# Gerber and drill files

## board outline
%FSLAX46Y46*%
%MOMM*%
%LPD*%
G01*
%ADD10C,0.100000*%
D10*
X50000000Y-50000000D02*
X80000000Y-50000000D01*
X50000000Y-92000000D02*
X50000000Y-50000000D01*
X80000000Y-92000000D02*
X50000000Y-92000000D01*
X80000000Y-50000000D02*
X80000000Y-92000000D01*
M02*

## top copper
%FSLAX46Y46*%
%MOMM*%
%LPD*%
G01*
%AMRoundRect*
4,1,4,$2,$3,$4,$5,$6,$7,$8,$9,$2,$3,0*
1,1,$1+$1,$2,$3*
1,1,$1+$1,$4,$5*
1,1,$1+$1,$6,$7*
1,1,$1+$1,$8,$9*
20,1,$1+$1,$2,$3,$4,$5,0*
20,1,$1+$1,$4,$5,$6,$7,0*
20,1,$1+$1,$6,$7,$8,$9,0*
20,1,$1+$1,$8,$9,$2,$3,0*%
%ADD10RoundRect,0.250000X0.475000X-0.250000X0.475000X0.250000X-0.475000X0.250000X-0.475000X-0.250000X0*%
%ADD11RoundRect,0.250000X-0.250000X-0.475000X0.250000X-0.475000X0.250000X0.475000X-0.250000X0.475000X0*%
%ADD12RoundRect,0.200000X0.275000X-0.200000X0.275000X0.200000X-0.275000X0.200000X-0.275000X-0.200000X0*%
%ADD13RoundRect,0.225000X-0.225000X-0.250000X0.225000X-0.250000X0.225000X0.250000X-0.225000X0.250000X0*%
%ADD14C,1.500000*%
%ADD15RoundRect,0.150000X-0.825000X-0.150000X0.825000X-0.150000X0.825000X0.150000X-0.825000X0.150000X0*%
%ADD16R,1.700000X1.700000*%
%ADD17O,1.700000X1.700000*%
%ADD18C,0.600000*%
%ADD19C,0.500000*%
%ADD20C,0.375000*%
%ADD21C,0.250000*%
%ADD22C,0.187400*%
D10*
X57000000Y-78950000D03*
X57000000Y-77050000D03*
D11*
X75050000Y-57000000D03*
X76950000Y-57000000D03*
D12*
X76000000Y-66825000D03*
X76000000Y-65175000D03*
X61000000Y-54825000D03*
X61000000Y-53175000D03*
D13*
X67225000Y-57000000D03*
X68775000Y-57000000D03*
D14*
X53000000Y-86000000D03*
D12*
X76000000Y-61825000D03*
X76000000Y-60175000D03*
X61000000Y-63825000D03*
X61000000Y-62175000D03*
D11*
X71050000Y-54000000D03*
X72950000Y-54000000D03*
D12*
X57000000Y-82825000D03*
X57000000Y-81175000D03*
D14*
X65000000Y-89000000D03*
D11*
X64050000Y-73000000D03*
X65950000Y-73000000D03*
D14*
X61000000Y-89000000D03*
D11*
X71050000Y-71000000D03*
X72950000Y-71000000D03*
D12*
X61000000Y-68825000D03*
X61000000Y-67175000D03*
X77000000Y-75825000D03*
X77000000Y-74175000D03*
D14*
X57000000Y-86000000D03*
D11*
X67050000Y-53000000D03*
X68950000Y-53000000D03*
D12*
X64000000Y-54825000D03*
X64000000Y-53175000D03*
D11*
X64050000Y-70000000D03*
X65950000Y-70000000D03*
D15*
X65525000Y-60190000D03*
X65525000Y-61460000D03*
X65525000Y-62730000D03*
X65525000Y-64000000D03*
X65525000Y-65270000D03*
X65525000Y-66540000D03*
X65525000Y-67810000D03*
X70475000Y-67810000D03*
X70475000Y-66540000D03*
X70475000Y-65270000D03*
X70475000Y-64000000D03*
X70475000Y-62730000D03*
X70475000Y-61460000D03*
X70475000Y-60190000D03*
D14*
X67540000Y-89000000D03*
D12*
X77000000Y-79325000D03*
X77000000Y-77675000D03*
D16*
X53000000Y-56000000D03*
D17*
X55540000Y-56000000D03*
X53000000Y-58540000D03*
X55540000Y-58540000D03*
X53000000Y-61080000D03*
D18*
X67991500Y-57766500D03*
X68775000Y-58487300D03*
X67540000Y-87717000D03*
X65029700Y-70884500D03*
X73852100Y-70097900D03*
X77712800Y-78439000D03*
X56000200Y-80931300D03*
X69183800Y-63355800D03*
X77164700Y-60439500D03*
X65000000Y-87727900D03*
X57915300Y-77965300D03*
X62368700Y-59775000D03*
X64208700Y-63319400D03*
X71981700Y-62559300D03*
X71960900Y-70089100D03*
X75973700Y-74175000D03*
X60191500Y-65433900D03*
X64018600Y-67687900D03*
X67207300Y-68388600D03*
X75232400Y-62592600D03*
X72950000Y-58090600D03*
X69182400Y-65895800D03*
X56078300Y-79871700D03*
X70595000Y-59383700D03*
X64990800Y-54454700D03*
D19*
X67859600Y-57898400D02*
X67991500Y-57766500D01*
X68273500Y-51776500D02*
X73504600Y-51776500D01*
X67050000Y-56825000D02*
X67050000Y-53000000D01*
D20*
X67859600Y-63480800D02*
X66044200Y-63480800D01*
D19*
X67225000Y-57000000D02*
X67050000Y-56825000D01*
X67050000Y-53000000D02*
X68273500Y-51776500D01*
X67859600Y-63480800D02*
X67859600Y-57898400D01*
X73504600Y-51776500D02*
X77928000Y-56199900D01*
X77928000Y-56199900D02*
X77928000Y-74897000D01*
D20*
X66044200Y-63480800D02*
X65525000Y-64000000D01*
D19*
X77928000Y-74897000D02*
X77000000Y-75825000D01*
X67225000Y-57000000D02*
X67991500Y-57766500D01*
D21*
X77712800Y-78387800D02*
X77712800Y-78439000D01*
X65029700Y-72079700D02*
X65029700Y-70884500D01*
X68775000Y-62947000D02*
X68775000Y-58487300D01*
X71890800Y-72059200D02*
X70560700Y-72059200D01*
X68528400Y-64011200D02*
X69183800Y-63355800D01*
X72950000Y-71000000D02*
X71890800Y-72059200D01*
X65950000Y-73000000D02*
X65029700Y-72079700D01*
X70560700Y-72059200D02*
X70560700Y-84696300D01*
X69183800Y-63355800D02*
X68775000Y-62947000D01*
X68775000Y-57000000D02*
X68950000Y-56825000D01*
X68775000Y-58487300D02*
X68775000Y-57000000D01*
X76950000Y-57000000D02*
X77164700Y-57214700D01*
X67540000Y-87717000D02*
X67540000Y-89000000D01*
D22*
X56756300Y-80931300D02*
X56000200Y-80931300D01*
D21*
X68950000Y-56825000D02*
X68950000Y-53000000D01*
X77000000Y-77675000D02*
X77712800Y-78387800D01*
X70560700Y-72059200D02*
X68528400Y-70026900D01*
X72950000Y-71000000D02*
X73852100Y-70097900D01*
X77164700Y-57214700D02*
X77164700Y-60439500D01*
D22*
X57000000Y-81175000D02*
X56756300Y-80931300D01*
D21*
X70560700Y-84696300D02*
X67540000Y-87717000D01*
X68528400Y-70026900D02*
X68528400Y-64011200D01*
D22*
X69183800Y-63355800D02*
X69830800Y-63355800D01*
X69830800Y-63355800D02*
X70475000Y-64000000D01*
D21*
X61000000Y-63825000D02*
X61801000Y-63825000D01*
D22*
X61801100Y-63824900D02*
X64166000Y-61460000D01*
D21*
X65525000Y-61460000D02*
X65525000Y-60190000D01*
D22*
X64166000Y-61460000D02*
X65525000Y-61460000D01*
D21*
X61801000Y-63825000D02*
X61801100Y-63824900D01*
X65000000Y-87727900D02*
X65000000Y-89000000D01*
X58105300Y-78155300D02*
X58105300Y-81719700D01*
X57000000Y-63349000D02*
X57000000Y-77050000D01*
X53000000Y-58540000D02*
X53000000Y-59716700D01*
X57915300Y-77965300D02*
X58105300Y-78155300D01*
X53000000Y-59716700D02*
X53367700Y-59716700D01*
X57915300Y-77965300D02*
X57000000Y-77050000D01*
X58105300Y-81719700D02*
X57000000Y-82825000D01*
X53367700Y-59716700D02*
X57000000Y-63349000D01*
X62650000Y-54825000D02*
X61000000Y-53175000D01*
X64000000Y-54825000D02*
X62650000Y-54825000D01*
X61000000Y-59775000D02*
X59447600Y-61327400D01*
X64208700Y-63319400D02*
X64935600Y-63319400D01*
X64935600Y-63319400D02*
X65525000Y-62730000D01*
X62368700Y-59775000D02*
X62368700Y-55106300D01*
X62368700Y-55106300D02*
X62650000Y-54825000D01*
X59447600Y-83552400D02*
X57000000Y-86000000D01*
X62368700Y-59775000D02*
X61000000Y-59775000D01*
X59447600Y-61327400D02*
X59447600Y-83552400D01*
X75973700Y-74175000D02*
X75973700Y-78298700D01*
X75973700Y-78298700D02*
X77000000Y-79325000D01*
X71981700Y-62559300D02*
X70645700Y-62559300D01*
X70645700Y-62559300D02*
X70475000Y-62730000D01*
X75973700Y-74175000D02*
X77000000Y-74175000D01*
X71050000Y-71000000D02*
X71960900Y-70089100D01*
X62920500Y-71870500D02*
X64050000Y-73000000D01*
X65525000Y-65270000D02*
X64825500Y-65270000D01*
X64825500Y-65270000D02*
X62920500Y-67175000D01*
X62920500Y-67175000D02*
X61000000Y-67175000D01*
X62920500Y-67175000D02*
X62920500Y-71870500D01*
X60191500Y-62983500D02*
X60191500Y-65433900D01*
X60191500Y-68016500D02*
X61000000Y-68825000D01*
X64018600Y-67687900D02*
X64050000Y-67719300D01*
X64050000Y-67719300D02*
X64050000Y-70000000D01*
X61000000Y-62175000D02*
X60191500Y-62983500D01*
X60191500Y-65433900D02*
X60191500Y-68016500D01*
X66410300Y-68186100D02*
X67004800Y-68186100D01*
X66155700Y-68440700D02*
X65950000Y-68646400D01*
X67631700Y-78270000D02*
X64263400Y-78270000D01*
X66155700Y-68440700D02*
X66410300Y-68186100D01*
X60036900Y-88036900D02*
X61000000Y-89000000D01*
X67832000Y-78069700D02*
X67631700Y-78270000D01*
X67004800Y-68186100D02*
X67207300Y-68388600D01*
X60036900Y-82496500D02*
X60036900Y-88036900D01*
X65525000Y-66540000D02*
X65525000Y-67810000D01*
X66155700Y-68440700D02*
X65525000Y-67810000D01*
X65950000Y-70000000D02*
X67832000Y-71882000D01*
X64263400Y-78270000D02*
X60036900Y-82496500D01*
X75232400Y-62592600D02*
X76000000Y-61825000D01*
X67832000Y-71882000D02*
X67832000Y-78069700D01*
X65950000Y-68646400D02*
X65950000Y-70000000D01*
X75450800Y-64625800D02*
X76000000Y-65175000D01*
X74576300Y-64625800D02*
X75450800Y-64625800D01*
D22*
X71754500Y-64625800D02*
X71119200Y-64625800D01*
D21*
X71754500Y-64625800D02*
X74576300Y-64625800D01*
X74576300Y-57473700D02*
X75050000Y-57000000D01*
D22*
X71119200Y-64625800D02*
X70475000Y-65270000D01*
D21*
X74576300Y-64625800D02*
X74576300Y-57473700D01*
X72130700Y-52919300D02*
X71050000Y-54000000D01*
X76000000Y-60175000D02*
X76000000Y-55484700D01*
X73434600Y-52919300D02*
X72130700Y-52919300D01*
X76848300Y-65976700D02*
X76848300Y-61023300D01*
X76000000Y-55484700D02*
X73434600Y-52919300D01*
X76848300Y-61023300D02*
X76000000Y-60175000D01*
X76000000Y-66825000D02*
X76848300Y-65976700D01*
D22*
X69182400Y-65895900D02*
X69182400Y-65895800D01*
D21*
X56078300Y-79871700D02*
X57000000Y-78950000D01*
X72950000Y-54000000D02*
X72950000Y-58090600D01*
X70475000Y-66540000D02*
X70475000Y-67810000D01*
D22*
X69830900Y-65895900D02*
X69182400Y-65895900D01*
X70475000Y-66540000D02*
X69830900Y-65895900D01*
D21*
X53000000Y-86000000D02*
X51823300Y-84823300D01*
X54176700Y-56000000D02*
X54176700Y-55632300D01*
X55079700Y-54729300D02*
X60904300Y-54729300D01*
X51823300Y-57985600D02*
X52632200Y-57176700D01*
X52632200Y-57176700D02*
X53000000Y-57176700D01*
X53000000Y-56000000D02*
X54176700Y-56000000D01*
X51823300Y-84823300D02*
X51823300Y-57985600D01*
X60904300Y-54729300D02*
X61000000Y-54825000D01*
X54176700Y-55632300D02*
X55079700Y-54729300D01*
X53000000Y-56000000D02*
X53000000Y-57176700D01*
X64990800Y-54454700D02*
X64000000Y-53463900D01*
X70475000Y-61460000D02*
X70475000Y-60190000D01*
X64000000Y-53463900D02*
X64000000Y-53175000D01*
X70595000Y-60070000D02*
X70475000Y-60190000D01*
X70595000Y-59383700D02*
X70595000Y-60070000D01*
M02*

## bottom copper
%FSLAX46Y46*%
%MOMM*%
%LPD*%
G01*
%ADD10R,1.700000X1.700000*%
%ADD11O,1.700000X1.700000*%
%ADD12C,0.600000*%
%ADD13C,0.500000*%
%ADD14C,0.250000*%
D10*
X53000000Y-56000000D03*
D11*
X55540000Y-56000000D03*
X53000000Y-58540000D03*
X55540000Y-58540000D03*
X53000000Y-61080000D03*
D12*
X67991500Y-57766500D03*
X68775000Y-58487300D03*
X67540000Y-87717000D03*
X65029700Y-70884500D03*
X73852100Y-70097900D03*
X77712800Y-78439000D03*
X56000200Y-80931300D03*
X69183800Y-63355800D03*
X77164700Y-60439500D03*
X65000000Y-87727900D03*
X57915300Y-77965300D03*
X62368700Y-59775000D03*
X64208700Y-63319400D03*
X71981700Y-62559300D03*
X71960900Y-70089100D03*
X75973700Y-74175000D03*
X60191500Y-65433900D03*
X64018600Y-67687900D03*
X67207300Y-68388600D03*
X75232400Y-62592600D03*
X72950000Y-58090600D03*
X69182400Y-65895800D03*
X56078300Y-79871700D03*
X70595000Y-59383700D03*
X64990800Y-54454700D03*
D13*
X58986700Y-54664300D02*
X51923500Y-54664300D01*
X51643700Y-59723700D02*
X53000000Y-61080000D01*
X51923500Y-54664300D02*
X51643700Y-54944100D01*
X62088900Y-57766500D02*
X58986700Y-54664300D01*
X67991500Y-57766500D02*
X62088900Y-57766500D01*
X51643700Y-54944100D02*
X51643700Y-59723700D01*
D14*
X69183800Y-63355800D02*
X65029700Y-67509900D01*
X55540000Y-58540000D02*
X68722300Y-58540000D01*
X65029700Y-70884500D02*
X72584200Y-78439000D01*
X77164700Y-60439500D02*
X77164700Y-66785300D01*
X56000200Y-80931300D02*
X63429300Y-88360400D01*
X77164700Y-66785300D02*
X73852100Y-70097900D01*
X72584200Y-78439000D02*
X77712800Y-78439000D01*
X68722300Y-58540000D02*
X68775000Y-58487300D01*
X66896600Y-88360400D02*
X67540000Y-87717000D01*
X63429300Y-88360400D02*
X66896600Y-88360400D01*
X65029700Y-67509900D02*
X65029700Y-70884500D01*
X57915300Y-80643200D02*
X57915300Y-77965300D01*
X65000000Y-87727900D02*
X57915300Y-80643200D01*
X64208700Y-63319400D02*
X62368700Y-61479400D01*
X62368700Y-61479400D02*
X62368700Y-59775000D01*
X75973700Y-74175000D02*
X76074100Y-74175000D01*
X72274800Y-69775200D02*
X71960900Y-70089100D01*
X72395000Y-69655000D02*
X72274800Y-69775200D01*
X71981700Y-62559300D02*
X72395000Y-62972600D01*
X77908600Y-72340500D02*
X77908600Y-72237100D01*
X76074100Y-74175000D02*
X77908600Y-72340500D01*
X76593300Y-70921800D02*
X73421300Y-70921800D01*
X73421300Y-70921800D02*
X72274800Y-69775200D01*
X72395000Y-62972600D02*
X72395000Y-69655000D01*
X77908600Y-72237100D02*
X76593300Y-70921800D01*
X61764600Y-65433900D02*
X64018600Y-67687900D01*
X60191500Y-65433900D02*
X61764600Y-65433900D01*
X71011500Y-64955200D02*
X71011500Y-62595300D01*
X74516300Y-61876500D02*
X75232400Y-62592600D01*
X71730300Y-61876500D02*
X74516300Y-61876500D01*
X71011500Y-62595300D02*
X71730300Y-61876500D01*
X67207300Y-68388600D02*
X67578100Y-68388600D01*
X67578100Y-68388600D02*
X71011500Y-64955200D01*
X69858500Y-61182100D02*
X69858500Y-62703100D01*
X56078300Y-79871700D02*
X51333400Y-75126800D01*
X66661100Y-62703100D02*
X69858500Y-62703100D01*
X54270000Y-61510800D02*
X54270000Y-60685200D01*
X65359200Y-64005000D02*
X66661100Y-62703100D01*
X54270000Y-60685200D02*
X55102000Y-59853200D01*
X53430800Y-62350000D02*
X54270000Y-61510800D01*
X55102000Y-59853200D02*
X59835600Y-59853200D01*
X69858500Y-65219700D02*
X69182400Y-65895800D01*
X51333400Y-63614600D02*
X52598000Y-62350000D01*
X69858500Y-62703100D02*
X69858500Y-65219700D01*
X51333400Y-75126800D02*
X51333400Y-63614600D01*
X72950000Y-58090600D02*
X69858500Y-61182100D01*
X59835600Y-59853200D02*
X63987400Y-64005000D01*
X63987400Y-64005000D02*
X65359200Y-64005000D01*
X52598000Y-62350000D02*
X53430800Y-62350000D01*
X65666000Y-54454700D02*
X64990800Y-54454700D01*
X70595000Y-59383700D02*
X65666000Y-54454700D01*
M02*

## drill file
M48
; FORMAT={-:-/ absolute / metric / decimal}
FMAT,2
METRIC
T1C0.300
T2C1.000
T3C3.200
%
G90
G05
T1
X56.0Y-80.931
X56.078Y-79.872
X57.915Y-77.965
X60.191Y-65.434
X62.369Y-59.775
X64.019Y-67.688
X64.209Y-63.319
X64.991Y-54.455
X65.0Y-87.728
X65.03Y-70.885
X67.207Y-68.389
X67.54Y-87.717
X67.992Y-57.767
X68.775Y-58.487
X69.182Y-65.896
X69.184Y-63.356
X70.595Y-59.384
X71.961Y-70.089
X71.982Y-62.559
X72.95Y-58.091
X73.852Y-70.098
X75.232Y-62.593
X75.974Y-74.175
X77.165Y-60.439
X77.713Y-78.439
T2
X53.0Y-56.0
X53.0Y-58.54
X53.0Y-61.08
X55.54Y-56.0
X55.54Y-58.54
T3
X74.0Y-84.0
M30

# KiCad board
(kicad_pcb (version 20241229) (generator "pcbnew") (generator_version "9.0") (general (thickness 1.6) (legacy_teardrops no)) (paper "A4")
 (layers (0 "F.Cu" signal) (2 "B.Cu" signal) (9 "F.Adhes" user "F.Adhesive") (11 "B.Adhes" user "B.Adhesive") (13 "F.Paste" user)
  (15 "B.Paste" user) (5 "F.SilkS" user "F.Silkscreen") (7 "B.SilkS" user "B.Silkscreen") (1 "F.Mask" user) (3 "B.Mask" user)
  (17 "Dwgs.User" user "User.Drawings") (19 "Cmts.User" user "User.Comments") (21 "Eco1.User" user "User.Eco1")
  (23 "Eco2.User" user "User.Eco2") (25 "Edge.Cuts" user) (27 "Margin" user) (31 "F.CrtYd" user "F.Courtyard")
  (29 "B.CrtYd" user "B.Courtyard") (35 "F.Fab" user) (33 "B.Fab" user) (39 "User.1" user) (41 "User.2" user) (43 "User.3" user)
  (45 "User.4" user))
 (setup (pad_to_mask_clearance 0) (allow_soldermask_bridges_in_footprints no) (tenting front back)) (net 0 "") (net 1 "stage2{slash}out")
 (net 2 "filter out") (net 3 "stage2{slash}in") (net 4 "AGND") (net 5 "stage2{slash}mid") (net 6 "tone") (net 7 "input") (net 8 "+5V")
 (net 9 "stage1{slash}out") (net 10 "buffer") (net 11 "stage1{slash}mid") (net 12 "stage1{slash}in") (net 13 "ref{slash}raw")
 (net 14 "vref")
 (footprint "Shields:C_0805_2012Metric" (layer "F.Cu") (at 57 78 90)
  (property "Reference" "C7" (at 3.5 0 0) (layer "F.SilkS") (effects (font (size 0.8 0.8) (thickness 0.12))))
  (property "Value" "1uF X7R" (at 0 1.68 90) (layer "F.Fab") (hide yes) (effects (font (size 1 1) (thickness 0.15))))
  (pad "1" smd roundrect (at -0.95 0 90) (size 1 1.45) (layers "F.Cu" "F.Mask" "F.Paste") (roundrect_rratio 0.25) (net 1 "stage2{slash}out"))
  (pad "2" smd roundrect (at 0.95 0 90) (size 1 1.45) (layers "F.Cu" "F.Mask" "F.Paste") (roundrect_rratio 0.25) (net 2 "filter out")))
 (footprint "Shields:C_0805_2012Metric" (layer "F.Cu") (at 76 57)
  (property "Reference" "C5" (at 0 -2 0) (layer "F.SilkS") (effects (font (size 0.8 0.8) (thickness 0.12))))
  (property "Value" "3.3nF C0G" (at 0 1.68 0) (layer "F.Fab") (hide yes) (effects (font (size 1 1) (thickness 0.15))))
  (pad "1" smd roundrect (at -0.95 0) (size 1 1.45) (layers "F.Cu" "F.Mask" "F.Paste") (roundrect_rratio 0.25) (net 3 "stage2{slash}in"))
  (pad "2" smd roundrect (at 0.95 0) (size 1 1.45) (layers "F.Cu" "F.Mask" "F.Paste") (roundrect_rratio 0.25) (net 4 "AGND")))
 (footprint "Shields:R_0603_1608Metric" (layer "F.Cu") (at 76 66 90)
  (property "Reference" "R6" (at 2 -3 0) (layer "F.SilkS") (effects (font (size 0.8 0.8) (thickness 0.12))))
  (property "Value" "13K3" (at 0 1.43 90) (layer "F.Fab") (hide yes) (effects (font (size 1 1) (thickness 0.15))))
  (pad "1" smd roundrect (at -0.825 0 90) (size 0.8 0.95) (layers "F.Cu" "F.Mask" "F.Paste") (roundrect_rratio 0.25)
   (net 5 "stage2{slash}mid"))
  (pad "2" smd roundrect (at 0.825 0 90) (size 0.8 0.95) (layers "F.Cu" "F.Mask" "F.Paste") (roundrect_rratio 0.25)
   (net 3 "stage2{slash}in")))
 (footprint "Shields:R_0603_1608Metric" (layer "F.Cu") (at 61 54 90)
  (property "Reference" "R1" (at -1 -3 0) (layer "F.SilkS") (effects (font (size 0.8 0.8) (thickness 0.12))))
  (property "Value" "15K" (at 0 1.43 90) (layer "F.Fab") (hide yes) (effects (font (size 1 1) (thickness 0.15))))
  (pad "1" smd roundrect (at -0.825 0 90) (size 0.8 0.95) (layers "F.Cu" "F.Mask" "F.Paste") (roundrect_rratio 0.25) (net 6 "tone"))
  (pad "2" smd roundrect (at 0.825 0 90) (size 0.8 0.95) (layers "F.Cu" "F.Mask" "F.Paste") (roundrect_rratio 0.25) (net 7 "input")))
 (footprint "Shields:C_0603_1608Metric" (layer "F.Cu") (at 68 57)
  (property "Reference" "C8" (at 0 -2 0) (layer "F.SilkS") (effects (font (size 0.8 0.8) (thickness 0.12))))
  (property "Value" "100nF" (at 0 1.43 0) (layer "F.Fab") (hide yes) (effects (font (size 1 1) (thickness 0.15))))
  (pad "1" smd roundrect (at -0.775 0) (size 0.9 0.95) (layers "F.Cu" "F.Mask" "F.Paste") (roundrect_rratio 0.25) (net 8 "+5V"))
  (pad "2" smd roundrect (at 0.775 0) (size 0.9 0.95) (layers "F.Cu" "F.Mask" "F.Paste") (roundrect_rratio 0.25) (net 4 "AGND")))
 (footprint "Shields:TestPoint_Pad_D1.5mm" (layer "F.Cu") (at 53 86)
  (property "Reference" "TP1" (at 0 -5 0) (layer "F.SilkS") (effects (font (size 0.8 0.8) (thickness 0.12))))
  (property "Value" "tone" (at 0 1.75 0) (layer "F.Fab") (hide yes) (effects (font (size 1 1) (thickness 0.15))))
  (pad "1" smd circle (at 0 0) (size 1.5 1.5) (layers "F.Cu" "F.Mask") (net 6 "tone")))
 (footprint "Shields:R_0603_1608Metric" (layer "F.Cu") (at 76 61 90)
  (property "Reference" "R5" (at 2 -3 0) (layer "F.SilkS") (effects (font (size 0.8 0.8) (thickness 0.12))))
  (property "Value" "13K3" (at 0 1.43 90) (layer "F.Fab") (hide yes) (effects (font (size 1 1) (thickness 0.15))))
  (pad "1" smd roundrect (at -0.825 0 90) (size 0.8 0.95) (layers "F.Cu" "F.Mask" "F.Paste") (roundrect_rratio 0.25)
   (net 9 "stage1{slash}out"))
  (pad "2" smd roundrect (at 0.825 0 90) (size 0.8 0.95) (layers "F.Cu" "F.Mask" "F.Paste") (roundrect_rratio 0.25)
   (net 5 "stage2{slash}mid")))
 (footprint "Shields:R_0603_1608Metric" (layer "F.Cu") (at 61 63 90)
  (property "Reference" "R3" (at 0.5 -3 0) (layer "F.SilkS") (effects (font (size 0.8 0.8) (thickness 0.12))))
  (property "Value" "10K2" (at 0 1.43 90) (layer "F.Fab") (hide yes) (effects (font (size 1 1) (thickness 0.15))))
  (pad "1" smd roundrect (at -0.825 0 90) (size 0.8 0.95) (layers "F.Cu" "F.Mask" "F.Paste") (roundrect_rratio 0.25) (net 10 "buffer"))
  (pad "2" smd roundrect (at 0.825 0 90) (size 0.8 0.95) (layers "F.Cu" "F.Mask" "F.Paste") (roundrect_rratio 0.25)
   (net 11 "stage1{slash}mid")))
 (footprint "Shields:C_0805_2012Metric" (layer "F.Cu") (at 72 54)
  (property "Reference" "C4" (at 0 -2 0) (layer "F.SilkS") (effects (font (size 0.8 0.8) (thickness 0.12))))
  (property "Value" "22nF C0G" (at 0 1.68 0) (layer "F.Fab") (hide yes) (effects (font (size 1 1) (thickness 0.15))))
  (pad "1" smd roundrect (at -0.95 0) (size 1 1.45) (layers "F.Cu" "F.Mask" "F.Paste") (roundrect_rratio 0.25) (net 5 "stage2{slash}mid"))
  (pad "2" smd roundrect (at 0.95 0) (size 1 1.45) (layers "F.Cu" "F.Mask" "F.Paste") (roundrect_rratio 0.25) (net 1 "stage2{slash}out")))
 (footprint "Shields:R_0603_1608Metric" (layer "F.Cu") (at 57 82 90)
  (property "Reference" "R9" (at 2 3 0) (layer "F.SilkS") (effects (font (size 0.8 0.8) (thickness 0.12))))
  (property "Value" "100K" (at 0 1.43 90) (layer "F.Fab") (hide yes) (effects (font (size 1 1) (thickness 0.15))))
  (pad "1" smd roundrect (at -0.825 0 90) (size 0.8 0.95) (layers "F.Cu" "F.Mask" "F.Paste") (roundrect_rratio 0.25) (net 2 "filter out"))
  (pad "2" smd roundrect (at 0.825 0 90) (size 0.8 0.95) (layers "F.Cu" "F.Mask" "F.Paste") (roundrect_rratio 0.25) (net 4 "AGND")))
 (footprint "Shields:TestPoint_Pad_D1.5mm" (layer "F.Cu") (at 65 89)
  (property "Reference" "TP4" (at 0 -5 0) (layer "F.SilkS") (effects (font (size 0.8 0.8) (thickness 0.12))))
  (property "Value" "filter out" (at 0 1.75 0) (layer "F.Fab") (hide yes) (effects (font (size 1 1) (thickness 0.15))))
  (pad "1" smd circle (at 0 0) (size 1.5 1.5) (layers "F.Cu" "F.Mask") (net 2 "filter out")))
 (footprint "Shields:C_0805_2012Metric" (layer "F.Cu") (at 65 73)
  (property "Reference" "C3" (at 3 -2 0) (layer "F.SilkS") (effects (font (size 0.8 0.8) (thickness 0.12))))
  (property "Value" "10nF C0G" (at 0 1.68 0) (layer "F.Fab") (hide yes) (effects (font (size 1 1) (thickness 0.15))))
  (pad "1" smd roundrect (at -0.95 0) (size 1 1.45) (layers "F.Cu" "F.Mask" "F.Paste") (roundrect_rratio 0.25) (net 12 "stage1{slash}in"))
  (pad "2" smd roundrect (at 0.95 0) (size 1 1.45) (layers "F.Cu" "F.Mask" "F.Paste") (roundrect_rratio 0.25) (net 4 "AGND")))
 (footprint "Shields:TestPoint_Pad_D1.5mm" (layer "F.Cu") (at 61 89)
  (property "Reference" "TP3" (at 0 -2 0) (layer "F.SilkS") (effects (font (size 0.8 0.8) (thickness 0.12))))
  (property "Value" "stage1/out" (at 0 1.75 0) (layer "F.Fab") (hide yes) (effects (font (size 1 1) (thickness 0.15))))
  (pad "1" smd circle (at 0 0) (size 1.5 1.5) (layers "F.Cu" "F.Mask") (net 9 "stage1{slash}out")))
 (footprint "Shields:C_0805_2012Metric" (layer "F.Cu") (at 72 71)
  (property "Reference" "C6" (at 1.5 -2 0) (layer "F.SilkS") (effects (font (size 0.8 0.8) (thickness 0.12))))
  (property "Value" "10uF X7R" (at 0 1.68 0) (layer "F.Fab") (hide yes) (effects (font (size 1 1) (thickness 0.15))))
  (pad "1" smd roundrect (at -0.95 0) (size 1 1.45) (layers "F.Cu" "F.Mask" "F.Paste") (roundrect_rratio 0.25) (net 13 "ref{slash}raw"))
  (pad "2" smd roundrect (at 0.95 0) (size 1 1.45) (layers "F.Cu" "F.Mask" "F.Paste") (roundrect_rratio 0.25) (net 4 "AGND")))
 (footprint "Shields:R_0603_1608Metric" (layer "F.Cu") (at 61 68 90)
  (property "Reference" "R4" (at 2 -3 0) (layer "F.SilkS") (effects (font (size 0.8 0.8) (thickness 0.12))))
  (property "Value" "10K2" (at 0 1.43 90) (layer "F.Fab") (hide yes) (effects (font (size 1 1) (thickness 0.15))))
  (pad "1" smd roundrect (at -0.825 0 90) (size 0.8 0.95) (layers "F.Cu" "F.Mask" "F.Paste") (roundrect_rratio 0.25)
   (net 11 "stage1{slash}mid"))
  (pad "2" smd roundrect (at 0.825 0 90) (size 0.8 0.95) (layers "F.Cu" "F.Mask" "F.Paste") (roundrect_rratio 0.25)
   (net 12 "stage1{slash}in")))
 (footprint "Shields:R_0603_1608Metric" (layer "F.Cu") (at 77 75 90)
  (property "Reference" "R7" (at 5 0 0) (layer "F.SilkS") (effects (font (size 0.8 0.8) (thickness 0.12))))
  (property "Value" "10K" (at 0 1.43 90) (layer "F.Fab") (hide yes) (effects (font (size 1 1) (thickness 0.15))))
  (pad "1" smd roundrect (at -0.825 0 90) (size 0.8 0.95) (layers "F.Cu" "F.Mask" "F.Paste") (roundrect_rratio 0.25) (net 8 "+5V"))
  (pad "2" smd roundrect (at 0.825 0 90) (size 0.8 0.95) (layers "F.Cu" "F.Mask" "F.Paste") (roundrect_rratio 0.25) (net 13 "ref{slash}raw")))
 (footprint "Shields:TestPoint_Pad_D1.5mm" (layer "F.Cu") (at 57 86)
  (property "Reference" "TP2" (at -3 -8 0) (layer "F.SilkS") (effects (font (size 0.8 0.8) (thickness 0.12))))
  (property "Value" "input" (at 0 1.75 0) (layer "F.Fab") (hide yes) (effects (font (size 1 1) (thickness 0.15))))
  (pad "1" smd circle (at 0 0) (size 1.5 1.5) (layers "F.Cu" "F.Mask") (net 7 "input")))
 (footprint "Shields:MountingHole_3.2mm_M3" (layer "F.Cu") (at 74 84)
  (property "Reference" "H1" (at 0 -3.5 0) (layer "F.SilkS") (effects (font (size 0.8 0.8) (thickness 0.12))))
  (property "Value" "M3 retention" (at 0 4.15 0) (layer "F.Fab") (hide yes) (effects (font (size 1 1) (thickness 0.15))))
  (pad "" np_thru_hole circle (at 0 0) (size 3.2 3.2) (drill 3.2) (layers "*.Cu" "*.Mask")))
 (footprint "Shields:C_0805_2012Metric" (layer "F.Cu") (at 68 53)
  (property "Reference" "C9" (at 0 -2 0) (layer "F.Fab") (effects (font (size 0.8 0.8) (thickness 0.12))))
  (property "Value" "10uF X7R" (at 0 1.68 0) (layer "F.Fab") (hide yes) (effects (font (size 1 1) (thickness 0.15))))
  (pad "1" smd roundrect (at -0.95 0) (size 1 1.45) (layers "F.Cu" "F.Mask" "F.Paste") (roundrect_rratio 0.25) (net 8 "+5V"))
  (pad "2" smd roundrect (at 0.95 0) (size 1 1.45) (layers "F.Cu" "F.Mask" "F.Paste") (roundrect_rratio 0.25) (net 4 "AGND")))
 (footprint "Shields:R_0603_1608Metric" (layer "F.Cu") (at 64 54 90)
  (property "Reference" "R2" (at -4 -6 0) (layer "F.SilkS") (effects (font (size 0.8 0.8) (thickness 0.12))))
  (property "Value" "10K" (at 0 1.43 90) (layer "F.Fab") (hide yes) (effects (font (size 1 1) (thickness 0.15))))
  (pad "1" smd roundrect (at -0.825 0 90) (size 0.8 0.95) (layers "F.Cu" "F.Mask" "F.Paste") (roundrect_rratio 0.25) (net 7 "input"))
  (pad "2" smd roundrect (at 0.825 0 90) (size 0.8 0.95) (layers "F.Cu" "F.Mask" "F.Paste") (roundrect_rratio 0.25) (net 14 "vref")))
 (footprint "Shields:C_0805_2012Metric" (layer "F.Cu") (at 65 70)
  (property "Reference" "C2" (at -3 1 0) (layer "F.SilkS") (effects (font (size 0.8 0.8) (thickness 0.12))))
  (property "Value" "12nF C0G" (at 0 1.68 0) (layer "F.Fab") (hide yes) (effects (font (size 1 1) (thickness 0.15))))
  (pad "1" smd roundrect (at -0.95 0) (size 1 1.45) (layers "F.Cu" "F.Mask" "F.Paste") (roundrect_rratio 0.25) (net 11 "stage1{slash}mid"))
  (pad "2" smd roundrect (at 0.95 0) (size 1 1.45) (layers "F.Cu" "F.Mask" "F.Paste") (roundrect_rratio 0.25) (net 9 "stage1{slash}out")))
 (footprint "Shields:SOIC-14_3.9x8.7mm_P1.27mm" (layer "F.Cu") (at 68 64)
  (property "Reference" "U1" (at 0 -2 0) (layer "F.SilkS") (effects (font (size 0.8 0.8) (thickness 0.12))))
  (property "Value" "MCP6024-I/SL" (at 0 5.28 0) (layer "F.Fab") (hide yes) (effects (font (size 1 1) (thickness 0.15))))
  (pad "1" smd roundrect (at -2.475 -3.81) (size 1.95 0.6) (layers "F.Cu" "F.Mask" "F.Paste") (roundrect_rratio 0.25) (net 10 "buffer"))
  (pad "2" smd roundrect (at -2.475 -2.54) (size 1.95 0.6) (layers "F.Cu" "F.Mask" "F.Paste") (roundrect_rratio 0.25) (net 10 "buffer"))
  (pad "3" smd roundrect (at -2.475 -1.27) (size 1.95 0.6) (layers "F.Cu" "F.Mask" "F.Paste") (roundrect_rratio 0.25) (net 7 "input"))
  (pad "4" smd roundrect (at -2.475 0) (size 1.95 0.6) (layers "F.Cu" "F.Mask" "F.Paste") (roundrect_rratio 0.25) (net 8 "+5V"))
  (pad "5" smd roundrect (at -2.475 1.27) (size 1.95 0.6) (layers "F.Cu" "F.Mask" "F.Paste") (roundrect_rratio 0.25)
   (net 12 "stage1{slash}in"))
  (pad "6" smd roundrect (at -2.475 2.54) (size 1.95 0.6) (layers "F.Cu" "F.Mask" "F.Paste") (roundrect_rratio 0.25)
   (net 9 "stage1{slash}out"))
  (pad "7" smd roundrect (at -2.475 3.81) (size 1.95 0.6) (layers "F.Cu" "F.Mask" "F.Paste") (roundrect_rratio 0.25)
   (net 9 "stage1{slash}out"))
  (pad "8" smd roundrect (at 2.475 3.81) (size 1.95 0.6) (layers "F.Cu" "F.Mask" "F.Paste") (roundrect_rratio 0.25)
   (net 1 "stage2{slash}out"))
  (pad "9" smd roundrect (at 2.475 2.54) (size 1.95 0.6) (layers "F.Cu" "F.Mask" "F.Paste") (roundrect_rratio 0.25)
   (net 1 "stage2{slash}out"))
  (pad "10" smd roundrect (at 2.475 1.27) (size 1.95 0.6) (layers "F.Cu" "F.Mask" "F.Paste") (roundrect_rratio 0.25)
   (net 3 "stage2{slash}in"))
  (pad "11" smd roundrect (at 2.475 0) (size 1.95 0.6) (layers "F.Cu" "F.Mask" "F.Paste") (roundrect_rratio 0.25) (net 4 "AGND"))
  (pad "12" smd roundrect (at 2.475 -1.27) (size 1.95 0.6) (layers "F.Cu" "F.Mask" "F.Paste") (roundrect_rratio 0.25)
   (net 13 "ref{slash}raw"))
  (pad "13" smd roundrect (at 2.475 -2.54) (size 1.95 0.6) (layers "F.Cu" "F.Mask" "F.Paste") (roundrect_rratio 0.25) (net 14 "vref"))
  (pad "14" smd roundrect (at 2.475 -3.81) (size 1.95 0.6) (layers "F.Cu" "F.Mask" "F.Paste") (roundrect_rratio 0.25) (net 14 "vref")))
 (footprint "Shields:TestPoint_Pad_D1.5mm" (layer "F.Cu") (at 67.54 89)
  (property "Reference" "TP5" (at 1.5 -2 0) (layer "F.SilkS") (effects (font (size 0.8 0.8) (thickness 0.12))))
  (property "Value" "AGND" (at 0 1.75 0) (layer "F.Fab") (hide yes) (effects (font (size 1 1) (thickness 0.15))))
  (pad "1" smd circle (at 0 0) (size 1.5 1.5) (layers "F.Cu" "F.Mask") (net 4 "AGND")))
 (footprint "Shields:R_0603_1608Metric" (layer "F.Cu") (at 77 78.5 90)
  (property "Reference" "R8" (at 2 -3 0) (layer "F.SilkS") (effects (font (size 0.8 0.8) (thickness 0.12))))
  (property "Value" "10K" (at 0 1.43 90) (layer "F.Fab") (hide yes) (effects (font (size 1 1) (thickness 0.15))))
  (pad "1" smd roundrect (at -0.825 0 90) (size 0.8 0.95) (layers "F.Cu" "F.Mask" "F.Paste") (roundrect_rratio 0.25)
   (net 13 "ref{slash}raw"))
  (pad "2" smd roundrect (at 0.825 0 90) (size 0.8 0.95) (layers "F.Cu" "F.Mask" "F.Paste") (roundrect_rratio 0.25) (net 4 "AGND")))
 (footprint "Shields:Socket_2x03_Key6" (layer "B.Cu") (at 53 56)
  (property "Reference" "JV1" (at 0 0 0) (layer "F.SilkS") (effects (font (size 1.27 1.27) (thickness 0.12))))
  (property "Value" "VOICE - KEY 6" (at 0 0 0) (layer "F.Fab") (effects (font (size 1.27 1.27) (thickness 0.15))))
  (pad "1" thru_hole rect (at 0 0) (size 1.7 1.7) (drill 1) (layers "*.Cu") (remove_unused_layers no) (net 6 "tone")
   (thermal_bridge_angle 45))
  (pad "2" thru_hole oval (at 2.54 0) (size 1.7 1.7) (drill 1) (layers "*.Cu") (remove_unused_layers no) (thermal_bridge_angle 45))
  (pad "3" thru_hole oval (at 0 2.54) (size 1.7 1.7) (drill 1) (layers "*.Cu") (remove_unused_layers no) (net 2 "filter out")
   (thermal_bridge_angle 45))
  (pad "4" thru_hole oval (at 2.54 2.54) (size 1.7 1.7) (drill 1) (layers "*.Cu") (remove_unused_layers no) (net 4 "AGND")
   (thermal_bridge_angle 45))
  (pad "5" thru_hole oval (at 0 5.08) (size 1.7 1.7) (drill 1) (layers "*.Cu") (remove_unused_layers no) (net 8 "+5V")
   (thermal_bridge_angle 45)))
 (gr_line (start 50 50) (end 80 50) (stroke (width 0.1) (type default)) (layer "Edge.Cuts"))
 (gr_line (start 50 92) (end 50 50) (stroke (width 0.1) (type default)) (layer "Edge.Cuts"))
 (gr_line (start 80 92) (end 50 92) (stroke (width 0.1) (type default)) (layer "Edge.Cuts"))
 (gr_line (start 80 50) (end 80 92) (stroke (width 0.1) (type default)) (layer "Edge.Cuts"))
 (segment (start 67.8596 57.8984) (end 67.9915 57.7665) (width 0.5) (layer "F.Cu") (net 8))
 (segment (start 68.2735 51.7765) (end 73.5046 51.7765) (width 0.5) (layer "F.Cu") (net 8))
 (segment (start 67.05 56.825) (end 67.05 53) (width 0.5) (layer "F.Cu") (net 8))
 (segment (start 67.8596 63.4808) (end 66.0442 63.4808) (width 0.375) (layer "F.Cu") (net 8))
 (segment (start 67.225 57) (end 67.05 56.825) (width 0.5) (layer "F.Cu") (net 8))
 (segment (start 67.05 53) (end 68.2735 51.7765) (width 0.5) (layer "F.Cu") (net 8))
 (segment (start 67.8596 63.4808) (end 67.8596 57.8984) (width 0.5) (layer "F.Cu") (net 8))
 (segment (start 73.5046 51.7765) (end 77.928 56.1999) (width 0.5) (layer "F.Cu") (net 8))
 (segment (start 77.928 56.1999) (end 77.928 74.897) (width 0.5) (layer "F.Cu") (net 8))
 (segment (start 66.0442 63.4808) (end 65.525 64) (width 0.375) (layer "F.Cu") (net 8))
 (segment (start 77.928 74.897) (end 77 75.825) (width 0.5) (layer "F.Cu") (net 8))
 (segment (start 67.225 57) (end 67.9915 57.7665) (width 0.5) (layer "F.Cu") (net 8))
 (via (at 67.9915 57.7665) (size 0.6) (drill 0.3) (layers "F.Cu" "B.Cu") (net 8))
 (segment (start 58.9867 54.6643) (end 51.9235 54.6643) (width 0.5) (layer "B.Cu") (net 8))
 (segment (start 51.6437 59.7237) (end 53 61.08) (width 0.5) (layer "B.Cu") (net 8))
 (segment (start 51.9235 54.6643) (end 51.6437 54.9441) (width 0.5) (layer "B.Cu") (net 8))
 (segment (start 62.0889 57.7665) (end 58.9867 54.6643) (width 0.5) (layer "B.Cu") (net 8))
 (segment (start 67.9915 57.7665) (end 62.0889 57.7665) (width 0.5) (layer "B.Cu") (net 8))
 (segment (start 51.6437 54.9441) (end 51.6437 59.7237) (width 0.5) (layer "B.Cu") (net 8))
 (segment (start 77.7128 78.3878) (end 77.7128 78.439) (width 0.25) (layer "F.Cu") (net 4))
 (segment (start 65.0297 72.0797) (end 65.0297 70.8845) (width 0.25) (layer "F.Cu") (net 4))
 (segment (start 68.775 62.947) (end 68.775 58.4873) (width 0.25) (layer "F.Cu") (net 4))
 (segment (start 71.8908 72.0592) (end 70.5607 72.0592) (width 0.25) (layer "F.Cu") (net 4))
 (segment (start 68.5284 64.0112) (end 69.1838 63.3558) (width 0.25) (layer "F.Cu") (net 4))
 (segment (start 72.95 71) (end 71.8908 72.0592) (width 0.25) (layer "F.Cu") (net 4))
 (segment (start 65.95 73) (end 65.0297 72.0797) (width 0.25) (layer "F.Cu") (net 4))
 (segment (start 70.5607 72.0592) (end 70.5607 84.6963) (width 0.25) (layer "F.Cu") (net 4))
 (segment (start 69.1838 63.3558) (end 68.775 62.947) (width 0.25) (layer "F.Cu") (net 4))
 (segment (start 68.775 57) (end 68.95 56.825) (width 0.25) (layer "F.Cu") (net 4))
 (segment (start 68.775 58.4873) (end 68.775 57) (width 0.25) (layer "F.Cu") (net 4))
 (segment (start 76.95 57) (end 77.1647 57.2147) (width 0.25) (layer "F.Cu") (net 4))
 (segment (start 67.54 87.717) (end 67.54 89) (width 0.25) (layer "F.Cu") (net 4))
 (segment (start 56.7563 80.9313) (end 56.0002 80.9313) (width 0.1874) (layer "F.Cu") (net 4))
 (segment (start 68.95 56.825) (end 68.95 53) (width 0.25) (layer "F.Cu") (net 4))
 (segment (start 77 77.675) (end 77.7128 78.3878) (width 0.25) (layer "F.Cu") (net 4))
 (segment (start 70.5607 72.0592) (end 68.5284 70.0269) (width 0.25) (layer "F.Cu") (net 4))
 (segment (start 72.95 71) (end 73.8521 70.0979) (width 0.25) (layer "F.Cu") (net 4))
 (segment (start 77.1647 57.2147) (end 77.1647 60.4395) (width 0.25) (layer "F.Cu") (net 4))
 (segment (start 57 81.175) (end 56.7563 80.9313) (width 0.1874) (layer "F.Cu") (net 4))
 (segment (start 70.5607 84.6963) (end 67.54 87.717) (width 0.25) (layer "F.Cu") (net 4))
 (segment (start 68.5284 70.0269) (end 68.5284 64.0112) (width 0.25) (layer "F.Cu") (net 4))
 (segment (start 69.1838 63.3558) (end 69.8308 63.3558) (width 0.1874) (layer "F.Cu") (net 4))
 (segment (start 69.8308 63.3558) (end 70.475 64) (width 0.1874) (layer "F.Cu") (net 4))
 (via (at 68.775 58.4873) (size 0.6) (drill 0.3) (layers "F.Cu" "B.Cu") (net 4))
 (via (at 67.54 87.717) (size 0.6) (drill 0.3) (layers "F.Cu" "B.Cu") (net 4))
 (via (at 65.0297 70.8845) (size 0.6) (drill 0.3) (layers "F.Cu" "B.Cu") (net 4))
 (via (at 73.8521 70.0979) (size 0.6) (drill 0.3) (layers "F.Cu" "B.Cu") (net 4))
 (via (at 77.7128 78.439) (size 0.6) (drill 0.3) (layers "F.Cu" "B.Cu") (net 4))
 (via (at 56.0002 80.9313) (size 0.6) (drill 0.3) (layers "F.Cu" "B.Cu") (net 4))
 (via (at 69.1838 63.3558) (size 0.6) (drill 0.3) (layers "F.Cu" "B.Cu") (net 4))
 (via (at 77.1647 60.4395) (size 0.6) (drill 0.3) (layers "F.Cu" "B.Cu") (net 4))
 (segment (start 69.1838 63.3558) (end 65.0297 67.5099) (width 0.25) (layer "B.Cu") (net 4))
 (segment (start 55.54 58.54) (end 68.7223 58.54) (width 0.25) (layer "B.Cu") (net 4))
 (segment (start 65.0297 70.8845) (end 72.5842 78.439) (width 0.25) (layer "B.Cu") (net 4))
 (segment (start 77.1647 60.4395) (end 77.1647 66.7853) (width 0.25) (layer "B.Cu") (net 4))
 (segment (start 56.0002 80.9313) (end 63.4293 88.3604) (width 0.25) (layer "B.Cu") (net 4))
 (segment (start 77.1647 66.7853) (end 73.8521 70.0979) (width 0.25) (layer "B.Cu") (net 4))
 (segment (start 72.5842 78.439) (end 77.7128 78.439) (width 0.25) (layer "B.Cu") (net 4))
 (segment (start 68.7223 58.54) (end 68.775 58.4873) (width 0.25) (layer "B.Cu") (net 4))
 (segment (start 66.8966 88.3604) (end 67.54 87.717) (width 0.25) (layer "B.Cu") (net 4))
 (segment (start 63.4293 88.3604) (end 66.8966 88.3604) (width 0.25) (layer "B.Cu") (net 4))
 (segment (start 65.0297 67.5099) (end 65.0297 70.8845) (width 0.25) (layer "B.Cu") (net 4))
 (segment (start 61 63.825) (end 61.801 63.825) (width 0.25) (layer "F.Cu") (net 10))
 (segment (start 61.8011 63.8249) (end 64.166 61.46) (width 0.1874) (layer "F.Cu") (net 10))
 (segment (start 65.525 61.46) (end 65.525 60.19) (width 0.25) (layer "F.Cu") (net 10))
 (segment (start 64.166 61.46) (end 65.525 61.46) (width 0.1874) (layer "F.Cu") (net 10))
 (segment (start 61.801 63.825) (end 61.8011 63.8249) (width 0.25) (layer "F.Cu") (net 10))
 (segment (start 65 87.7279) (end 65 89) (width 0.25) (layer "F.Cu") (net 2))
 (segment (start 58.1053 78.1553) (end 58.1053 81.7197) (width 0.25) (layer "F.Cu") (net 2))
 (segment (start 57 63.349) (end 57 77.05) (width 0.25) (layer "F.Cu") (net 2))
 (segment (start 53 58.54) (end 53 59.7167) (width 0.25) (layer "F.Cu") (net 2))
 (segment (start 57.9153 77.9653) (end 58.1053 78.1553) (width 0.25) (layer "F.Cu") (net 2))
 (segment (start 53 59.7167) (end 53.3677 59.7167) (width 0.25) (layer "F.Cu") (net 2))
 (segment (start 57.9153 77.9653) (end 57 77.05) (width 0.25) (layer "F.Cu") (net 2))
 (segment (start 58.1053 81.7197) (end 57 82.825) (width 0.25) (layer "F.Cu") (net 2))
 (segment (start 53.3677 59.7167) (end 57 63.349) (width 0.25) (layer "F.Cu") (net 2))
 (via (at 65 87.7279) (size 0.6) (drill 0.3) (layers "F.Cu" "B.Cu") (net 2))
 (via (at 57.9153 77.9653) (size 0.6) (drill 0.3) (layers "F.Cu" "B.Cu") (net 2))
 (segment (start 57.9153 80.6432) (end 57.9153 77.9653) (width 0.25) (layer "B.Cu") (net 2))
 (segment (start 65 87.7279) (end 57.9153 80.6432) (width 0.25) (layer "B.Cu") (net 2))
 (segment (start 62.65 54.825) (end 61 53.175) (width 0.25) (layer "F.Cu") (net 7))
 (segment (start 64 54.825) (end 62.65 54.825) (width 0.25) (layer "F.Cu") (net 7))
 (segment (start 61 59.775) (end 59.4476 61.3274) (width 0.25) (layer "F.Cu") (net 7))
 (segment (start 64.2087 63.3194) (end 64.9356 63.3194) (width 0.25) (layer "F.Cu") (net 7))
 (segment (start 64.9356 63.3194) (end 65.525 62.73) (width 0.25) (layer "F.Cu") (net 7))
 (segment (start 62.3687 59.775) (end 62.3687 55.1063) (width 0.25) (layer "F.Cu") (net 7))
 (segment (start 62.3687 55.1063) (end 62.65 54.825) (width 0.25) (layer "F.Cu") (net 7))
 (segment (start 59.4476 83.5524) (end 57 86) (width 0.25) (layer "F.Cu") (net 7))
 (segment (start 62.3687 59.775) (end 61 59.775) (width 0.25) (layer "F.Cu") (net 7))
 (segment (start 59.4476 61.3274) (end 59.4476 83.5524) (width 0.25) (layer "F.Cu") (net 7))
 (via (at 62.3687 59.775) (size 0.6) (drill 0.3) (layers "F.Cu" "B.Cu") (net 7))
 (via (at 64.2087 63.3194) (size 0.6) (drill 0.3) (layers "F.Cu" "B.Cu") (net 7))
 (segment (start 64.2087 63.3194) (end 62.3687 61.4794) (width 0.25) (layer "B.Cu") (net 7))
 (segment (start 62.3687 61.4794) (end 62.3687 59.775) (width 0.25) (layer "B.Cu") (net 7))
 (segment (start 75.9737 74.175) (end 75.9737 78.2987) (width 0.25) (layer "F.Cu") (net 13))
 (segment (start 75.9737 78.2987) (end 77 79.325) (width 0.25) (layer "F.Cu") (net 13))
 (segment (start 71.9817 62.5593) (end 70.6457 62.5593) (width 0.25) (layer "F.Cu") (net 13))
 (segment (start 70.6457 62.5593) (end 70.475 62.73) (width 0.25) (layer "F.Cu") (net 13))
 (segment (start 75.9737 74.175) (end 77 74.175) (width 0.25) (layer "F.Cu") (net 13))
 (segment (start 71.05 71) (end 71.9609 70.0891) (width 0.25) (layer "F.Cu") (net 13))
 (via (at 71.9817 62.5593) (size 0.6) (drill 0.3) (layers "F.Cu" "B.Cu") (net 13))
 (via (at 71.9609 70.0891) (size 0.6) (drill 0.3) (layers "F.Cu" "B.Cu") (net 13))
 (via (at 75.9737 74.175) (size 0.6) (drill 0.3) (layers "F.Cu" "B.Cu") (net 13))
 (segment (start 75.9737 74.175) (end 76.0741 74.175) (width 0.25) (layer "B.Cu") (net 13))
 (segment (start 72.2748 69.7752) (end 71.9609 70.0891) (width 0.25) (layer "B.Cu") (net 13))
 (segment (start 72.395 69.655) (end 72.2748 69.7752) (width 0.25) (layer "B.Cu") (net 13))
 (segment (start 71.9817 62.5593) (end 72.395 62.9726) (width 0.25) (layer "B.Cu") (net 13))
 (segment (start 77.9086 72.3405) (end 77.9086 72.2371) (width 0.25) (layer "B.Cu") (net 13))
 (segment (start 76.0741 74.175) (end 77.9086 72.3405) (width 0.25) (layer "B.Cu") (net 13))
 (segment (start 76.5933 70.9218) (end 73.4213 70.9218) (width 0.25) (layer "B.Cu") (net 13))
 (segment (start 73.4213 70.9218) (end 72.2748 69.7752) (width 0.25) (layer "B.Cu") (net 13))
 (segment (start 72.395 62.9726) (end 72.395 69.655) (width 0.25) (layer "B.Cu") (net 13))
 (segment (start 77.9086 72.2371) (end 76.5933 70.9218) (width 0.25) (layer "B.Cu") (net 13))
 (segment (start 62.9205 71.8705) (end 64.05 73) (width 0.25) (layer "F.Cu") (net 12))
 (segment (start 65.525 65.27) (end 64.8255 65.27) (width 0.25) (layer "F.Cu") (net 12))
 (segment (start 64.8255 65.27) (end 62.9205 67.175) (width 0.25) (layer "F.Cu") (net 12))
 (segment (start 62.9205 67.175) (end 61 67.175) (width 0.25) (layer "F.Cu") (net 12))
 (segment (start 62.9205 67.175) (end 62.9205 71.8705) (width 0.25) (layer "F.Cu") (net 12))
 (segment (start 60.1915 62.9835) (end 60.1915 65.4339) (width 0.25) (layer "F.Cu") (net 11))
 (segment (start 60.1915 68.0165) (end 61 68.825) (width 0.25) (layer "F.Cu") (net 11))
 (segment (start 64.0186 67.6879) (end 64.05 67.7193) (width 0.25) (layer "F.Cu") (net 11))
 (segment (start 64.05 67.7193) (end 64.05 70) (width 0.25) (layer "F.Cu") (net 11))
 (segment (start 61 62.175) (end 60.1915 62.9835) (width 0.25) (layer "F.Cu") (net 11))
 (segment (start 60.1915 65.4339) (end 60.1915 68.0165) (width 0.25) (layer "F.Cu") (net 11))
 (via (at 60.1915 65.4339) (size 0.6) (drill 0.3) (layers "F.Cu" "B.Cu") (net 11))
 (via (at 64.0186 67.6879) (size 0.6) (drill 0.3) (layers "F.Cu" "B.Cu") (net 11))
 (segment (start 61.7646 65.4339) (end 64.0186 67.6879) (width 0.25) (layer "B.Cu") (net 11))
 (segment (start 60.1915 65.4339) (end 61.7646 65.4339) (width 0.25) (layer "B.Cu") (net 11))
 (segment (start 66.4103 68.1861) (end 67.0048 68.1861) (width 0.25) (layer "F.Cu") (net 9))
 (segment (start 66.1557 68.4407) (end 65.95 68.6464) (width 0.25) (layer "F.Cu") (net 9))
 (segment (start 67.6317 78.27) (end 64.2634 78.27) (width 0.25) (layer "F.Cu") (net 9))
 (segment (start 66.1557 68.4407) (end 66.4103 68.1861) (width 0.25) (layer "F.Cu") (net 9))
 (segment (start 60.0369 88.0369) (end 61 89) (width 0.25) (layer "F.Cu") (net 9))
 (segment (start 67.832 78.0697) (end 67.6317 78.27) (width 0.25) (layer "F.Cu") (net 9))
 (segment (start 67.0048 68.1861) (end 67.2073 68.3886) (width 0.25) (layer "F.Cu") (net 9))
 (segment (start 60.0369 82.4965) (end 60.0369 88.0369) (width 0.25) (layer "F.Cu") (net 9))
 (segment (start 65.525 66.54) (end 65.525 67.81) (width 0.25) (layer "F.Cu") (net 9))
 (segment (start 66.1557 68.4407) (end 65.525 67.81) (width 0.25) (layer "F.Cu") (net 9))
 (segment (start 65.95 70) (end 67.832 71.882) (width 0.25) (layer "F.Cu") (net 9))
 (segment (start 64.2634 78.27) (end 60.0369 82.4965) (width 0.25) (layer "F.Cu") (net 9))
 (segment (start 75.2324 62.5926) (end 76 61.825) (width 0.25) (layer "F.Cu") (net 9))
 (segment (start 67.832 71.882) (end 67.832 78.0697) (width 0.25) (layer "F.Cu") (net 9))
 (segment (start 65.95 68.6464) (end 65.95 70) (width 0.25) (layer "F.Cu") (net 9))
 (via (at 67.2073 68.3886) (size 0.6) (drill 0.3) (layers "F.Cu" "B.Cu") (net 9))
 (via (at 75.2324 62.5926) (size 0.6) (drill 0.3) (layers "F.Cu" "B.Cu") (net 9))
 (segment (start 71.0115 64.9552) (end 71.0115 62.5953) (width 0.25) (layer "B.Cu") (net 9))
 (segment (start 74.5163 61.8765) (end 75.2324 62.5926) (width 0.25) (layer "B.Cu") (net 9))
 (segment (start 71.7303 61.8765) (end 74.5163 61.8765) (width 0.25) (layer "B.Cu") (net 9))
 (segment (start 71.0115 62.5953) (end 71.7303 61.8765) (width 0.25) (layer "B.Cu") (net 9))
 (segment (start 67.2073 68.3886) (end 67.5781 68.3886) (width 0.25) (layer "B.Cu") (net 9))
 (segment (start 67.5781 68.3886) (end 71.0115 64.9552) (width 0.25) (layer "B.Cu") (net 9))
 (segment (start 75.4508 64.6258) (end 76 65.175) (width 0.25) (layer "F.Cu") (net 3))
 (segment (start 74.5763 64.6258) (end 75.4508 64.6258) (width 0.25) (layer "F.Cu") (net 3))
 (segment (start 71.7545 64.6258) (end 71.1192 64.6258) (width 0.1874) (layer "F.Cu") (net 3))
 (segment (start 71.7545 64.6258) (end 74.5763 64.6258) (width 0.25) (layer "F.Cu") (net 3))
 (segment (start 74.5763 57.4737) (end 75.05 57) (width 0.25) (layer "F.Cu") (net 3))
 (segment (start 71.1192 64.6258) (end 70.475 65.27) (width 0.1874) (layer "F.Cu") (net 3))
 (segment (start 74.5763 64.6258) (end 74.5763 57.4737) (width 0.25) (layer "F.Cu") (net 3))
 (segment (start 72.1307 52.9193) (end 71.05 54) (width 0.25) (layer "F.Cu") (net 5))
 (segment (start 76 60.175) (end 76 55.4847) (width 0.25) (layer "F.Cu") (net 5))
 (segment (start 73.4346 52.9193) (end 72.1307 52.9193) (width 0.25) (layer "F.Cu") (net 5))
 (segment (start 76.8483 65.9767) (end 76.8483 61.0233) (width 0.25) (layer "F.Cu") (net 5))
 (segment (start 76 55.4847) (end 73.4346 52.9193) (width 0.25) (layer "F.Cu") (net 5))
 (segment (start 76.8483 61.0233) (end 76 60.175) (width 0.25) (layer "F.Cu") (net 5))
 (segment (start 76 66.825) (end 76.8483 65.9767) (width 0.25) (layer "F.Cu") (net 5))
 (segment (start 69.1824 65.8959) (end 69.1824 65.8958) (width 0.1874) (layer "F.Cu") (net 1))
 (segment (start 56.0783 79.8717) (end 57 78.95) (width 0.25) (layer "F.Cu") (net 1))
 (segment (start 72.95 54) (end 72.95 58.0906) (width 0.25) (layer "F.Cu") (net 1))
 (segment (start 70.475 66.54) (end 70.475 67.81) (width 0.25) (layer "F.Cu") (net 1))
 (segment (start 69.8309 65.8959) (end 69.1824 65.8959) (width 0.1874) (layer "F.Cu") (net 1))
 (segment (start 70.475 66.54) (end 69.8309 65.8959) (width 0.1874) (layer "F.Cu") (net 1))
 (via (at 72.95 58.0906) (size 0.6) (drill 0.3) (layers "F.Cu" "B.Cu") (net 1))
 (via (at 69.1824 65.8958) (size 0.6) (drill 0.3) (layers "F.Cu" "B.Cu") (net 1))
 (via (at 56.0783 79.8717) (size 0.6) (drill 0.3) (layers "F.Cu" "B.Cu") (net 1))
 (segment (start 69.8585 61.1821) (end 69.8585 62.7031) (width 0.25) (layer "B.Cu") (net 1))
 (segment (start 56.0783 79.8717) (end 51.3334 75.1268) (width 0.25) (layer "B.Cu") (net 1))
 (segment (start 66.6611 62.7031) (end 69.8585 62.7031) (width 0.25) (layer "B.Cu") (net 1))
 (segment (start 54.27 61.5108) (end 54.27 60.6852) (width 0.25) (layer "B.Cu") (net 1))
 (segment (start 65.3592 64.005) (end 66.6611 62.7031) (width 0.25) (layer "B.Cu") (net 1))
 (segment (start 54.27 60.6852) (end 55.102 59.8532) (width 0.25) (layer "B.Cu") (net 1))
 (segment (start 53.4308 62.35) (end 54.27 61.5108) (width 0.25) (layer "B.Cu") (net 1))
 (segment (start 55.102 59.8532) (end 59.8356 59.8532) (width 0.25) (layer "B.Cu") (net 1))
 (segment (start 69.8585 65.2197) (end 69.1824 65.8958) (width 0.25) (layer "B.Cu") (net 1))
 (segment (start 51.3334 63.6146) (end 52.598 62.35) (width 0.25) (layer "B.Cu") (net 1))
 (segment (start 69.8585 62.7031) (end 69.8585 65.2197) (width 0.25) (layer "B.Cu") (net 1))
 (segment (start 51.3334 75.1268) (end 51.3334 63.6146) (width 0.25) (layer "B.Cu") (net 1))
 (segment (start 72.95 58.0906) (end 69.8585 61.1821) (width 0.25) (layer "B.Cu") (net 1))
 (segment (start 59.8356 59.8532) (end 63.9874 64.005) (width 0.25) (layer "B.Cu") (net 1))
 (segment (start 63.9874 64.005) (end 65.3592 64.005) (width 0.25) (layer "B.Cu") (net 1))
 (segment (start 52.598 62.35) (end 53.4308 62.35) (width 0.25) (layer "B.Cu") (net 1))
 (segment (start 53 86) (end 51.8233 84.8233) (width 0.25) (layer "F.Cu") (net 6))
 (segment (start 54.1767 56) (end 54.1767 55.6323) (width 0.25) (layer "F.Cu") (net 6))
 (segment (start 55.0797 54.7293) (end 60.9043 54.7293) (width 0.25) (layer "F.Cu") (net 6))
 (segment (start 51.8233 57.9856) (end 52.6322 57.1767) (width 0.25) (layer "F.Cu") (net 6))
 (segment (start 52.6322 57.1767) (end 53 57.1767) (width 0.25) (layer "F.Cu") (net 6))
 (segment (start 53 56) (end 54.1767 56) (width 0.25) (layer "F.Cu") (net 6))
 (segment (start 51.8233 84.8233) (end 51.8233 57.9856) (width 0.25) (layer "F.Cu") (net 6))
 (segment (start 60.9043 54.7293) (end 61 54.825) (width 0.25) (layer "F.Cu") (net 6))
 (segment (start 54.1767 55.6323) (end 55.0797 54.7293) (width 0.25) (layer "F.Cu") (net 6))
 (segment (start 53 56) (end 53 57.1767) (width 0.25) (layer "F.Cu") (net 6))
 (segment (start 64.9908 54.4547) (end 64 53.4639) (width 0.25) (layer "F.Cu") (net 14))
 (segment (start 70.475 61.46) (end 70.475 60.19) (width 0.25) (layer "F.Cu") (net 14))
 (segment (start 64 53.4639) (end 64 53.175) (width 0.25) (layer "F.Cu") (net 14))
 (segment (start 70.595 60.07) (end 70.475 60.19) (width 0.25) (layer "F.Cu") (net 14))
 (segment (start 70.595 59.3837) (end 70.595 60.07) (width 0.25) (layer "F.Cu") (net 14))
 (via (at 70.595 59.3837) (size 0.6) (drill 0.3) (layers "F.Cu" "B.Cu") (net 14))
 (via (at 64.9908 54.4547) (size 0.6) (drill 0.3) (layers "F.Cu" "B.Cu") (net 14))
 (segment (start 65.666 54.4547) (end 64.9908 54.4547) (width 0.25) (layer "B.Cu") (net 14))
 (segment (start 70.595 59.3837) (end 65.666 54.4547) (width 0.25) (layer "B.Cu") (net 14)))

